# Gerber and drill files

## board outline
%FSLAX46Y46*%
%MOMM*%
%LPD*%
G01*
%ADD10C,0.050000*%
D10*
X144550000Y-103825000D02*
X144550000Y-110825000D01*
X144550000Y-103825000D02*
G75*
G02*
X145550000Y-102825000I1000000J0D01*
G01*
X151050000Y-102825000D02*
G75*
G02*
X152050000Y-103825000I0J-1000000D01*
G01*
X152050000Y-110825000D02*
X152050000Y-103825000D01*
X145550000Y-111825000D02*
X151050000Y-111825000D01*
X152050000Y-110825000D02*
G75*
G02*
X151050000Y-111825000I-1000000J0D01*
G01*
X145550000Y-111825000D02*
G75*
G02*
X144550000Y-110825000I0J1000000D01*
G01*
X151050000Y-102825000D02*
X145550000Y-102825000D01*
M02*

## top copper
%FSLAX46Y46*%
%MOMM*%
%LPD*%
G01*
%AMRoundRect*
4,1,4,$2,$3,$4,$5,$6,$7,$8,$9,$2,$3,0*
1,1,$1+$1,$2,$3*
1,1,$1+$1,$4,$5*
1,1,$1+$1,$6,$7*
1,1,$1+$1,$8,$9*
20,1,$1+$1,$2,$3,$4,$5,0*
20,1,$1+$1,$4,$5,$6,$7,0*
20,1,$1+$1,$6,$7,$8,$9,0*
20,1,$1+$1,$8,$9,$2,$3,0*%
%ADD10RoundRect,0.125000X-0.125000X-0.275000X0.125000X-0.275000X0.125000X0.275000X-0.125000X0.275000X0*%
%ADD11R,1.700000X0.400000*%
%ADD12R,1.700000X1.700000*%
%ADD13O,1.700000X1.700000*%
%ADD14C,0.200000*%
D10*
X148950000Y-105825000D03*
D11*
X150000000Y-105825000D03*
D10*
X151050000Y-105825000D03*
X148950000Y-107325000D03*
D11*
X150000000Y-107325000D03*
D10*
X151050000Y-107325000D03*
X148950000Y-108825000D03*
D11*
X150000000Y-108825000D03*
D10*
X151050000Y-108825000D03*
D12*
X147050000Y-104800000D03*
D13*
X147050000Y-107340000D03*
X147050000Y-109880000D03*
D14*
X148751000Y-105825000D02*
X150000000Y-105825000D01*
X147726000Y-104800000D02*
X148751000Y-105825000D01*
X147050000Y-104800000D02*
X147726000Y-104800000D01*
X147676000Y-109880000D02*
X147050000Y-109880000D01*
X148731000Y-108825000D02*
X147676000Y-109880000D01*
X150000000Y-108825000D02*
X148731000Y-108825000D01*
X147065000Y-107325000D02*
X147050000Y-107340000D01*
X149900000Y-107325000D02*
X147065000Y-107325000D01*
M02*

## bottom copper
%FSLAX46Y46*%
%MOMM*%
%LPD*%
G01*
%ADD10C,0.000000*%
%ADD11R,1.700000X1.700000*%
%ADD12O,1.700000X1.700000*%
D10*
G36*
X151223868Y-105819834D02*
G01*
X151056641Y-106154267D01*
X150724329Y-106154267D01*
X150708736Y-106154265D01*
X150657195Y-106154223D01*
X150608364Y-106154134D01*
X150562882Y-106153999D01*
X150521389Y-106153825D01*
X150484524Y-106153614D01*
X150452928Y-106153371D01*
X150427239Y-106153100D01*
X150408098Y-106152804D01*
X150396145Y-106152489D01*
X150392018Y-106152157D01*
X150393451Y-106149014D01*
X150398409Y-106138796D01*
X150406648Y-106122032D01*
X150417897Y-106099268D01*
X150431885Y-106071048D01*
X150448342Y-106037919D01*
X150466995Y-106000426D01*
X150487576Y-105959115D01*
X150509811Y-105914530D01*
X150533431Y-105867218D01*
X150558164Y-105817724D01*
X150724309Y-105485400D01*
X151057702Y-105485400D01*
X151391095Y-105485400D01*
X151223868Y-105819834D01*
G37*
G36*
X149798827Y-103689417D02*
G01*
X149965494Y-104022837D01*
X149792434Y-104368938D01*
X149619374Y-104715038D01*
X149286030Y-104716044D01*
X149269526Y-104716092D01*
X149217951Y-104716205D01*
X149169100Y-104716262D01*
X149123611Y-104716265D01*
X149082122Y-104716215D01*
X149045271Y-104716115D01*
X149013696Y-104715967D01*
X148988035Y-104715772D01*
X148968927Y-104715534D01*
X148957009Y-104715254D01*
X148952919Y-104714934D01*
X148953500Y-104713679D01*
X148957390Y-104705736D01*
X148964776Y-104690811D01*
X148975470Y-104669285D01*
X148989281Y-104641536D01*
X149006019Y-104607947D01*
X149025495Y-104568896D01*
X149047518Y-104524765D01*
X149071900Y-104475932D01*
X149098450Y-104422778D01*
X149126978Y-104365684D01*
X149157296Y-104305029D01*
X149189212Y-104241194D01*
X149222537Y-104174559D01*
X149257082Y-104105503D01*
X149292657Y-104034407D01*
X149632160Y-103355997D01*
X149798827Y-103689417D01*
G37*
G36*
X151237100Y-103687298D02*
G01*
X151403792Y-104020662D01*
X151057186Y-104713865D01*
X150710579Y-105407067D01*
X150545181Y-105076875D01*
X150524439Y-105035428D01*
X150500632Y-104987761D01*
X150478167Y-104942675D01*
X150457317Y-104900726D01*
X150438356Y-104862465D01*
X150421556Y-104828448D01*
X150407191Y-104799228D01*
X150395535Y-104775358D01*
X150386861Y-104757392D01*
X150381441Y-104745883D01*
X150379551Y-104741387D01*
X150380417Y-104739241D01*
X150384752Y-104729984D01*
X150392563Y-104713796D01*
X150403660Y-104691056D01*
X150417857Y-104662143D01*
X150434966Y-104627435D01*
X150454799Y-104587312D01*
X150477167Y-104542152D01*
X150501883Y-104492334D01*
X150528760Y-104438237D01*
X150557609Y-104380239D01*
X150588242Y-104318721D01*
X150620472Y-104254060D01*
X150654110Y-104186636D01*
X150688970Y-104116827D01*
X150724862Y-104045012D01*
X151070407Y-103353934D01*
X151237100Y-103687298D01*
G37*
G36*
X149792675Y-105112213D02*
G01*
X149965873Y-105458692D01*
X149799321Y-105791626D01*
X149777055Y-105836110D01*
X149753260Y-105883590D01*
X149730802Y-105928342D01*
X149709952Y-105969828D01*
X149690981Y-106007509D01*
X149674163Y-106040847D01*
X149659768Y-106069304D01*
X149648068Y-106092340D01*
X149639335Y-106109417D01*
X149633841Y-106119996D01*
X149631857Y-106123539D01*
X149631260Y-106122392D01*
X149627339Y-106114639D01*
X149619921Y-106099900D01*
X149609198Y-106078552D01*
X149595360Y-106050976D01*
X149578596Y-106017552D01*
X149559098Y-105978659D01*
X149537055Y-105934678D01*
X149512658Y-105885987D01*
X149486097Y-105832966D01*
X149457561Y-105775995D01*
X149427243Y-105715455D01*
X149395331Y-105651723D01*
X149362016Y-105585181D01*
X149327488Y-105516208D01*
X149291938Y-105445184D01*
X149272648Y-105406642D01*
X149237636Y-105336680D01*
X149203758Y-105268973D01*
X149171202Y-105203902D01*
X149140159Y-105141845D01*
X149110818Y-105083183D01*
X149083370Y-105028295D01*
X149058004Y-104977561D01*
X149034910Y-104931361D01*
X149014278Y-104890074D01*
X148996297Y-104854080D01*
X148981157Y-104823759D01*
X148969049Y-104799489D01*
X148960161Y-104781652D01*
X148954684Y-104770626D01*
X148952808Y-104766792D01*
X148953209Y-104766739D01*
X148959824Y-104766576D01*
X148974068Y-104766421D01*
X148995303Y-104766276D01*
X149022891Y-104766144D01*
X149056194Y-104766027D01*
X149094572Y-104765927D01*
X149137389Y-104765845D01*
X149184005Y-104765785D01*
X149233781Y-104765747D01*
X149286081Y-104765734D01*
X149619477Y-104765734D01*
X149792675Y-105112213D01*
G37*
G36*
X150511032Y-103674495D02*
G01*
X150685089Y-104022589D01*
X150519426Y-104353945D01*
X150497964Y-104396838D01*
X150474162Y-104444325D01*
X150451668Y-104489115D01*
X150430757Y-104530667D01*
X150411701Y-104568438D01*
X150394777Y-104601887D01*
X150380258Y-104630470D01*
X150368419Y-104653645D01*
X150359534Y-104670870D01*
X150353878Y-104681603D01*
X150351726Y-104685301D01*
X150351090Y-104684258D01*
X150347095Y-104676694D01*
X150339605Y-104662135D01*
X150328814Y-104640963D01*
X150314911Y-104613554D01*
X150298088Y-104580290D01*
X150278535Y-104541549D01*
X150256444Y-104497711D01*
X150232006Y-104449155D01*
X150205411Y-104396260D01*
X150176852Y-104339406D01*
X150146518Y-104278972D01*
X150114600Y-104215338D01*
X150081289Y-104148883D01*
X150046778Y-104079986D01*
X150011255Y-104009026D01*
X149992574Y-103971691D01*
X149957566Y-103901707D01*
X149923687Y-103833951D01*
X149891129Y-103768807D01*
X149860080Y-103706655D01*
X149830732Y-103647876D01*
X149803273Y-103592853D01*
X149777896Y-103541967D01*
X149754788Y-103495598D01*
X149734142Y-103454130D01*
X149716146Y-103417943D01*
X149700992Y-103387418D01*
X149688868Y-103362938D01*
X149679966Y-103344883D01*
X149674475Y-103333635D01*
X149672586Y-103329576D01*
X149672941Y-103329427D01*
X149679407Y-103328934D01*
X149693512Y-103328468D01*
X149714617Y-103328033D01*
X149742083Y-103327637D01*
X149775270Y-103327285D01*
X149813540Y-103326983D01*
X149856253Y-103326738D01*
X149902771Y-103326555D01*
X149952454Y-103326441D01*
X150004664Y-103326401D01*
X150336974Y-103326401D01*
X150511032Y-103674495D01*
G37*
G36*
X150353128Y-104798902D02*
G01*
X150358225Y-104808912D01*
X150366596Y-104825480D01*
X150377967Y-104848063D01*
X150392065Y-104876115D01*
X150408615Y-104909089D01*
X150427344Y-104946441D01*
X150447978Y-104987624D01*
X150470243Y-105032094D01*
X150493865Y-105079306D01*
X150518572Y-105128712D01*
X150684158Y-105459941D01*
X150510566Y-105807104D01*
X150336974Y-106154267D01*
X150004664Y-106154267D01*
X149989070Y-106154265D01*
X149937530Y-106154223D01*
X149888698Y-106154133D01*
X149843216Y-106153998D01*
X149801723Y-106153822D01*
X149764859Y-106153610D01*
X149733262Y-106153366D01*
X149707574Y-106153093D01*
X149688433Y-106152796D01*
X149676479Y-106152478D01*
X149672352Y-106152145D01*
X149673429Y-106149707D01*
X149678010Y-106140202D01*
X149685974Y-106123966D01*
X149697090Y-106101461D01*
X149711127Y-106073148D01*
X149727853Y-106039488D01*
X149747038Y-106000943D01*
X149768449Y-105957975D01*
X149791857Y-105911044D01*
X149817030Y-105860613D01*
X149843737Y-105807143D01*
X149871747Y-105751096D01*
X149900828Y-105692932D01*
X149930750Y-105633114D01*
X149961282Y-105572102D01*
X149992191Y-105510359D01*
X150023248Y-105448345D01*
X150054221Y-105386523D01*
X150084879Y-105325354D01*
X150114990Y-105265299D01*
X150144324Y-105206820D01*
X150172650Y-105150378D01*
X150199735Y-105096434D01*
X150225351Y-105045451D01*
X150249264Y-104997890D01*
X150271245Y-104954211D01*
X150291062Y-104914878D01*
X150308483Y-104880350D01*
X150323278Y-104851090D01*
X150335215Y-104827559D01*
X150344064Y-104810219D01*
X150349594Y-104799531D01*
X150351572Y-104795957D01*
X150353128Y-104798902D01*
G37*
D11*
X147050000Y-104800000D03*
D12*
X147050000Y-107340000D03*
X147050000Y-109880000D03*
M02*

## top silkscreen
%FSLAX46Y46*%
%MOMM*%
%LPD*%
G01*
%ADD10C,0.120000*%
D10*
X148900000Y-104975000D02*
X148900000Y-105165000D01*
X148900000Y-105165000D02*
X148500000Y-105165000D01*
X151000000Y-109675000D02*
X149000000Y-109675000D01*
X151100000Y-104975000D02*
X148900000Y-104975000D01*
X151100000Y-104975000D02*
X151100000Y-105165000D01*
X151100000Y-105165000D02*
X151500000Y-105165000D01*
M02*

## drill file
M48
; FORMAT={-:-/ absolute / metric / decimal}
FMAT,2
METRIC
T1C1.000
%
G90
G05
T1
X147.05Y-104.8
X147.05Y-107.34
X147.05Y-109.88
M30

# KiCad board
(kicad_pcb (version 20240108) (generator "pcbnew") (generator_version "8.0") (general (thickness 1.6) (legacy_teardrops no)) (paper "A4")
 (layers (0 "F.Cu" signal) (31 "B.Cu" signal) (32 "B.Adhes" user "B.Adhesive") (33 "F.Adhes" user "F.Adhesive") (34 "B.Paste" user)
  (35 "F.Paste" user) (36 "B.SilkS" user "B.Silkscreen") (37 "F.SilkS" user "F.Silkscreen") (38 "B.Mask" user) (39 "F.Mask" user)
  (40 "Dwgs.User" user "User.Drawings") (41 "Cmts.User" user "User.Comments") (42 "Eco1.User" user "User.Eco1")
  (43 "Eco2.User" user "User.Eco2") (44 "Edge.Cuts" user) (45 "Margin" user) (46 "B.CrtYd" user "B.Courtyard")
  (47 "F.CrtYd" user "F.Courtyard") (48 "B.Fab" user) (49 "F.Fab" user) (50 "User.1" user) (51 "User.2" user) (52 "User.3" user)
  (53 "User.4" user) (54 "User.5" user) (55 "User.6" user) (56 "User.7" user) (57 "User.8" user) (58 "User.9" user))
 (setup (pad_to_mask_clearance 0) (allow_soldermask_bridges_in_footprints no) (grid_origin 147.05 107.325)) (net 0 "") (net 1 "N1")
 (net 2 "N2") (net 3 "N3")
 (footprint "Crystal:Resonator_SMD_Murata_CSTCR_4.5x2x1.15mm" (layer "F.Cu") (at 150 107.325)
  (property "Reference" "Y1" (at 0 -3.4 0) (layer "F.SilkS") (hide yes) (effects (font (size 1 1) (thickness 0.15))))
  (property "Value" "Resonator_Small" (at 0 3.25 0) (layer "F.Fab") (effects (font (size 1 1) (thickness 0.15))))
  (fp_line (start -1.1 -2.35) (end -1.1 -2.16) (stroke (width 0.12) (type default)) (layer "F.SilkS"))
  (fp_line (start -1.1 -2.16) (end -1.5 -2.16) (stroke (width 0.12) (type default)) (layer "F.SilkS"))
  (fp_line (start 1 2.35) (end -1 2.35) (stroke (width 0.12) (type solid)) (layer "F.SilkS"))
  (fp_line (start 1.1 -2.35) (end -1.1 -2.35) (stroke (width 0.12) (type solid)) (layer "F.SilkS"))
  (fp_line (start 1.1 -2.35) (end 1.1 -2.16) (stroke (width 0.12) (type default)) (layer "F.SilkS"))
  (fp_line (start 1.1 -2.16) (end 1.5 -2.16) (stroke (width 0.12) (type default)) (layer "F.SilkS"))
  (pad "1" smd roundrect (at -1.05 -1.5) (size 0.5 0.8) (layers "F.Cu" "F.Paste" "F.Mask") (roundrect_rratio 0.25) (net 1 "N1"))
  (pad "1" smd rect (at 0 -1.5 270) (size 0.4 1.7) (layers "F.Cu" "F.Paste" "F.Mask") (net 1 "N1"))
  (pad "1" smd roundrect (at 1.05 -1.5) (size 0.5 0.8) (layers "F.Cu" "F.Paste" "F.Mask") (roundrect_rratio 0.25) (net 1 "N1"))
  (pad "2" smd roundrect (at -1.05 0) (size 0.5 0.8) (layers "F.Cu" "F.Paste" "F.Mask") (roundrect_rratio 0.25) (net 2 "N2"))
  (pad "2" smd rect (at 0 0 270) (size 0.4 1.7) (layers "F.Cu" "F.Paste" "F.Mask") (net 2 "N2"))
  (pad "2" smd roundrect (at 1.05 0) (size 0.5 0.8) (layers "F.Cu" "F.Paste" "F.Mask") (roundrect_rratio 0.25) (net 2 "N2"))
  (pad "3" smd roundrect (at -1.05 1.5) (size 0.5 0.8) (layers "F.Cu" "F.Paste" "F.Mask") (roundrect_rratio 0.25) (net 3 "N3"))
  (pad "3" smd rect (at 0 1.5 270) (size 0.4 1.7) (layers "F.Cu" "F.Paste" "F.Mask") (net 3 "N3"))
  (pad "3" smd roundrect (at 1.05 1.5) (size 0.5 0.8) (layers "F.Cu" "F.Paste" "F.Mask") (roundrect_rratio 0.25) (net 3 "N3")))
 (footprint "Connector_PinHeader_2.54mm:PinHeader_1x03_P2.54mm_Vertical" (layer "B.Cu") (at 147.05 104.8 180)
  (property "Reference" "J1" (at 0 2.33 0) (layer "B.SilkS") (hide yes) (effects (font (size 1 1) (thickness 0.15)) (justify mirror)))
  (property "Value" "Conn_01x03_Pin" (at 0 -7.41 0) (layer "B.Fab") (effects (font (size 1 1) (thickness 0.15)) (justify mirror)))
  (pad "1" thru_hole rect (at 0 0 180) (size 1.7 1.7) (drill 1) (layers "*.Cu" "*.Mask") (remove_unused_layers no) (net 1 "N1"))
  (pad "2" thru_hole oval (at 0 -2.54 180) (size 1.7 1.7) (drill 1) (layers "*.Cu" "*.Mask") (remove_unused_layers no) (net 2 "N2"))
  (pad "3" thru_hole oval (at 0 -5.08 180) (size 1.7 1.7) (drill 1) (layers "*.Cu" "*.Mask") (remove_unused_layers no) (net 3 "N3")))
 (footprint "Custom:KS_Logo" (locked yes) (layer "B.Cu") (at 150.05 104.825 90)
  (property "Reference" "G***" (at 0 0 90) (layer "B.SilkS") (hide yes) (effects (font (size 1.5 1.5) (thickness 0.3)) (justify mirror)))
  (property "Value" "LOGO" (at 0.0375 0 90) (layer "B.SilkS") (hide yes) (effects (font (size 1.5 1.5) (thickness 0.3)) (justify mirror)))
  (fp_poly
   (pts (xy -0.6604 1.007702) (xy -0.6604 0.674309) (xy -0.992724 0.508164) (xy -1.042218 0.483431) (xy -1.08953 0.459811)
    (xy -1.134115 0.437576) (xy -1.175426 0.416995) (xy -1.212919 0.398342) (xy -1.246048 0.381885) (xy -1.274268 0.367897)
    (xy -1.297032 0.356648) (xy -1.313796 0.348409) (xy -1.324014 0.343451) (xy -1.327157 0.342018) (xy -1.327489 0.346145)
    (xy -1.327804 0.358098) (xy -1.3281 0.377239) (xy -1.328371 0.402928) (xy -1.328614 0.434524) (xy -1.328825 0.471389)
    (xy -1.328999 0.512882) (xy -1.329134 0.558364) (xy -1.329223 0.607195) (xy -1.329265 0.658736) (xy -1.329267 0.674329)
    (xy -1.329267 1.006641) (xy -0.994834 1.173868) (xy -0.6604 1.341095))
   (stroke (width 0) (type solid)) (fill solid) (layer "B.Cu"))
  (fp_poly
   (pts (xy 1.135583 -0.251173) (xy 1.469003 -0.41784) (xy 0.790593 -0.757343) (xy 0.719497 -0.792918) (xy 0.650441 -0.827463)
    (xy 0.583806 -0.860788) (xy 0.519971 -0.892704) (xy 0.459316 -0.923022) (xy 0.402222 -0.95155) (xy 0.349068 -0.9781)
    (xy 0.300235 -1.002482) (xy 0.256104 -1.024505) (xy 0.217053 -1.043981) (xy 0.183464 -1.060719) (xy 0.155715 -1.07453)
    (xy 0.134189 -1.085224) (xy 0.119264 -1.09261) (xy 0.111321 -1.0965) (xy 0.110066 -1.097081) (xy 0.109746 -1.092991)
    (xy 0.109466 -1.081073) (xy 0.109228 -1.061965) (xy 0.109033 -1.036304) (xy 0.108885 -1.004729) (xy 0.108785 -0.967878)
    (xy 0.108735 -0.926389) (xy 0.108738 -0.8809) (xy 0.108795 -0.832049) (xy 0.108908 -0.780474) (xy 0.108956 -0.76397)
    (xy 0.109962 -0.430626) (xy 0.456062 -0.257566) (xy 0.802163 -0.084506))
   (stroke (width 0) (type solid)) (fill solid) (layer "B.Cu"))
  (fp_poly
   (pts (xy 1.137702 1.1871) (xy 1.471066 1.020407) (xy 0.779988 0.674862) (xy 0.708173 0.63897) (xy 0.638364 0.60411) (xy 0.57094 0.570472)
    (xy 0.506279 0.538242) (xy 0.444761 0.507609) (xy 0.386763 0.47876) (xy 0.332666 0.451883) (xy 0.282848 0.427167) (xy 0.237688 0.404799)
    (xy 0.197565 0.384966) (xy 0.162857 0.367857) (xy 0.133944 0.35366) (xy 0.111204 0.342563) (xy 0.095016 0.334752) (xy 0.085759 0.330417)
    (xy 0.083613 0.329551) (xy 0.079117 0.331441) (xy 0.067608 0.336861) (xy 0.049642 0.345535) (xy 0.025772 0.357191)
    (xy -0.003448 0.371556) (xy -0.037465 0.388356) (xy -0.075726 0.407317) (xy -0.117675 0.428167) (xy -0.162761 0.450632)
    (xy -0.210428 0.474439) (xy -0.251875 0.495181) (xy -0.582067 0.660579) (xy 0.111135 1.007186) (xy 0.804338 1.353792))
   (stroke (width 0) (type solid)) (fill solid) (layer "B.Cu"))
  (fp_poly
   (pts (xy -0.287213 -0.257325) (xy 0.059266 -0.430523) (xy 0.059266 -0.763919) (xy 0.059253 -0.816219) (xy 0.059215 -0.865995)
    (xy 0.059155 -0.912611) (xy 0.059073 -0.955428) (xy 0.058973 -0.993806) (xy 0.058856 -1.027109) (xy 0.058724 -1.054697)
    (xy 0.058579 -1.075932) (xy 0.058424 -1.090176) (xy 0.058261 -1.096791) (xy 0.058208 -1.097192) (xy 0.054374 -1.095316)
    (xy 0.043348 -1.089839) (xy 0.025511 -1.080951) (xy 0.001241 -1.068843) (xy -0.02908 -1.053703) (xy -0.065074 -1.035722)
    (xy -0.106361 -1.01509) (xy -0.152561 -0.991996) (xy -0.203295 -0.96663) (xy -0.258183 -0.939182) (xy -0.316845 -0.909841)
    (xy -0.378902 -0.878798) (xy -0.443973 -0.846242) (xy -0.51168 -0.812364) (xy -0.581642 -0.777352) (xy -0.620184 -0.758062)
    (xy -0.691208 -0.722512) (xy -0.760181 -0.687984) (xy -0.826723 -0.654669) (xy -0.890455 -0.622757) (xy -0.950995 -0.592439)
    (xy -1.007966 -0.563903) (xy -1.060987 -0.537342) (xy -1.109678 -0.512945) (xy -1.153659 -0.490902) (xy -1.192552 -0.471404)
    (xy -1.225976 -0.45464) (xy -1.253552 -0.440802) (xy -1.2749 -0.430079) (xy -1.289639 -0.422661) (xy -1.297392 -0.41874)
    (xy -1.298539 -0.418143) (xy -1.294996 -0.416159) (xy -1.284417 -0.410665) (xy -1.26734 -0.401932) (xy -1.244304 -0.390232)
    (xy -1.215847 -0.375837) (xy -1.182509 -0.359019) (xy -1.144828 -0.340048) (xy -1.103342 -0.319198) (xy -1.05859 -0.29674)
    (xy -1.01111 -0.272945) (xy -0.966626 -0.250679) (xy -0.633692 -0.084127))
   (stroke (width 0) (type solid)) (fill solid) (layer "B.Cu"))
  (fp_poly
   (pts (xy 1.150505 0.461032) (xy 1.498599 0.286974) (xy 1.498599 -0.045336) (xy 1.498559 -0.097546) (xy 1.498445 -0.147229)
    (xy 1.498262 -0.193747) (xy 1.498017 -0.23646) (xy 1.497715 -0.27473) (xy 1.497363 -0.307917) (xy 1.496967 -0.335383)
    (xy 1.496532 -0.356488) (xy 1.496066 -0.370593) (xy 1.495573 -0.377059) (xy 1.495424 -0.377414) (xy 1.491365 -0.375525)
    (xy 1.480117 -0.370034) (xy 1.462062 -0.361132) (xy 1.437582 -0.349008) (xy 1.407057 -0.333854) (xy 1.37087 -0.315858)
    (xy 1.329402 -0.295212) (xy 1.283033 -0.272104) (xy 1.232147 -0.246727) (xy 1.177124 -0.219268) (xy 1.118345 -0.18992)
    (xy 1.056193 -0.158871) (xy 0.991049 -0.126313) (xy 0.923293 -0.092434) (xy 0.853309 -0.057426) (xy 0.815974 -0.038745)
    (xy 0.745014 -0.003222) (xy 0.676117 0.031289) (xy 0.609662 0.0646) (xy 0.546028 0.096518) (xy 0.485594 0.126852) (xy 0.42874 0.155411)
    (xy 0.375845 0.182006) (xy 0.327289 0.206444) (xy 0.283451 0.228535) (xy 0.24471 0.248088) (xy 0.211446 0.264911) (xy 0.184037 0.278814)
    (xy 0.162865 0.289605) (xy 0.148306 0.297095) (xy 0.140742 0.30109) (xy 0.139699 0.301726) (xy 0.143397 0.303878) (xy 0.15413 0.309534)
    (xy 0.171355 0.318419) (xy 0.19453 0.330258) (xy 0.223113 0.344777) (xy 0.256562 0.361701) (xy 0.294333 0.380757) (xy 0.335885 0.401668)
    (xy 0.380675 0.424162) (xy 0.428162 0.447964) (xy 0.471055 0.469426) (xy 0.802411 0.635089))
   (stroke (width 0) (type solid)) (fill solid) (layer "B.Cu"))
  (fp_poly
   (pts (xy -0.303712 0.468572) (xy -0.254306 0.443865) (xy -0.207094 0.420243) (xy -0.162624 0.397978) (xy -0.121441 0.377344)
    (xy -0.084089 0.358615) (xy -0.051115 0.342065) (xy -0.023063 0.327967) (xy -0.00048 0.316596) (xy 0.016088 0.308225)
    (xy 0.026098 0.303128) (xy 0.029043 0.301572) (xy 0.025469 0.299594) (xy 0.014781 0.294064) (xy -0.002559 0.285215)
    (xy -0.02609 0.273278) (xy -0.05535 0.258483) (xy -0.089878 0.241062) (xy -0.129211 0.221245) (xy -0.17289 0.199264)
    (xy -0.220451 0.175351) (xy -0.271434 0.149735) (xy -0.325378 0.12265) (xy -0.38182 0.094324) (xy -0.440299 0.06499)
    (xy -0.500354 0.034879) (xy -0.561523 0.004221) (xy -0.623345 -0.026752) (xy -0.685359 -0.057809) (xy -0.747102 -0.088718)
    (xy -0.808114 -0.11925) (xy -0.867932 -0.149172) (xy -0.926096 -0.178253) (xy -0.982143 -0.206263) (xy -1.035613 -0.23297)
    (xy -1.086044 -0.258143) (xy -1.132975 -0.281551) (xy -1.175943 -0.302962) (xy -1.214488 -0.322147) (xy -1.248148 -0.338873)
    (xy -1.276461 -0.35291) (xy -1.298966 -0.364026) (xy -1.315202 -0.37199) (xy -1.324707 -0.376571) (xy -1.327145 -0.377648)
    (xy -1.327478 -0.373521) (xy -1.327796 -0.361567) (xy -1.328093 -0.342426) (xy -1.328366 -0.316738) (xy -1.32861 -0.285141)
    (xy -1.328822 -0.248277) (xy -1.328998 -0.206784) (xy -1.329133 -0.161302) (xy -1.329223 -0.11247) (xy -1.329265 -0.06093)
    (xy -1.329267 -0.045336) (xy -1.329267 0.286974) (xy -0.982104 0.460566) (xy -0.634941 0.634158))
   (stroke (width 0) (type solid)) (fill solid) (layer "B.Cu")))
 (gr_line (start 144.55 103.825) (end 144.55 110.825) (stroke (width 0.05) (type default)) (layer "Edge.Cuts"))
 (gr_arc (start 144.55 103.825) (mid 144.842893 103.117893) (end 145.55 102.825) (stroke (width 0.05) (type default)) (layer "Edge.Cuts"))
 (gr_arc (start 151.05 102.825) (mid 151.757107 103.117893) (end 152.05 103.825) (stroke (width 0.05) (type default)) (layer "Edge.Cuts"))
 (gr_line (start 152.05 110.825) (end 152.05 103.825) (stroke (width 0.05) (type default)) (layer "Edge.Cuts"))
 (gr_line (start 145.55 111.825) (end 151.05 111.825) (stroke (width 0.05) (type default)) (layer "Edge.Cuts"))
 (gr_arc (start 152.05 110.825) (mid 151.757107 111.532107) (end 151.05 111.825) (stroke (width 0.05) (type default)) (layer "Edge.Cuts"))
 (gr_arc (start 145.55 111.825) (mid 144.842893 111.532107) (end 144.55 110.825) (stroke (width 0.05) (type default)) (layer "Edge.Cuts"))
 (gr_line (start 151.05 102.825) (end 145.55 102.825) (stroke (width 0.05) (type default)) (layer "Edge.Cuts"))
 (segment (start 148.751 105.825) (end 150 105.825) (width 0.2) (layer "F.Cu") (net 1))
 (segment (start 147.726 104.8) (end 148.751 105.825) (width 0.2) (layer "F.Cu") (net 1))
 (segment (start 147.05 104.8) (end 147.726 104.8) (width 0.2) (layer "F.Cu") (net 1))
 (segment (start 147.676 109.88) (end 147.05 109.88) (width 0.2) (layer "F.Cu") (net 3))
 (segment (start 148.731 108.825) (end 147.676 109.88) (width 0.2) (layer "F.Cu") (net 3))
 (segment (start 150 108.825) (end 148.731 108.825) (width 0.2) (layer "F.Cu") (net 3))
 (segment (start 147.065 107.325) (end 147.05 107.34) (width 0.2) (layer "F.Cu") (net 2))
 (segment (start 149.9 107.325) (end 147.065 107.325) (width 0.2) (layer "F.Cu") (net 2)))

